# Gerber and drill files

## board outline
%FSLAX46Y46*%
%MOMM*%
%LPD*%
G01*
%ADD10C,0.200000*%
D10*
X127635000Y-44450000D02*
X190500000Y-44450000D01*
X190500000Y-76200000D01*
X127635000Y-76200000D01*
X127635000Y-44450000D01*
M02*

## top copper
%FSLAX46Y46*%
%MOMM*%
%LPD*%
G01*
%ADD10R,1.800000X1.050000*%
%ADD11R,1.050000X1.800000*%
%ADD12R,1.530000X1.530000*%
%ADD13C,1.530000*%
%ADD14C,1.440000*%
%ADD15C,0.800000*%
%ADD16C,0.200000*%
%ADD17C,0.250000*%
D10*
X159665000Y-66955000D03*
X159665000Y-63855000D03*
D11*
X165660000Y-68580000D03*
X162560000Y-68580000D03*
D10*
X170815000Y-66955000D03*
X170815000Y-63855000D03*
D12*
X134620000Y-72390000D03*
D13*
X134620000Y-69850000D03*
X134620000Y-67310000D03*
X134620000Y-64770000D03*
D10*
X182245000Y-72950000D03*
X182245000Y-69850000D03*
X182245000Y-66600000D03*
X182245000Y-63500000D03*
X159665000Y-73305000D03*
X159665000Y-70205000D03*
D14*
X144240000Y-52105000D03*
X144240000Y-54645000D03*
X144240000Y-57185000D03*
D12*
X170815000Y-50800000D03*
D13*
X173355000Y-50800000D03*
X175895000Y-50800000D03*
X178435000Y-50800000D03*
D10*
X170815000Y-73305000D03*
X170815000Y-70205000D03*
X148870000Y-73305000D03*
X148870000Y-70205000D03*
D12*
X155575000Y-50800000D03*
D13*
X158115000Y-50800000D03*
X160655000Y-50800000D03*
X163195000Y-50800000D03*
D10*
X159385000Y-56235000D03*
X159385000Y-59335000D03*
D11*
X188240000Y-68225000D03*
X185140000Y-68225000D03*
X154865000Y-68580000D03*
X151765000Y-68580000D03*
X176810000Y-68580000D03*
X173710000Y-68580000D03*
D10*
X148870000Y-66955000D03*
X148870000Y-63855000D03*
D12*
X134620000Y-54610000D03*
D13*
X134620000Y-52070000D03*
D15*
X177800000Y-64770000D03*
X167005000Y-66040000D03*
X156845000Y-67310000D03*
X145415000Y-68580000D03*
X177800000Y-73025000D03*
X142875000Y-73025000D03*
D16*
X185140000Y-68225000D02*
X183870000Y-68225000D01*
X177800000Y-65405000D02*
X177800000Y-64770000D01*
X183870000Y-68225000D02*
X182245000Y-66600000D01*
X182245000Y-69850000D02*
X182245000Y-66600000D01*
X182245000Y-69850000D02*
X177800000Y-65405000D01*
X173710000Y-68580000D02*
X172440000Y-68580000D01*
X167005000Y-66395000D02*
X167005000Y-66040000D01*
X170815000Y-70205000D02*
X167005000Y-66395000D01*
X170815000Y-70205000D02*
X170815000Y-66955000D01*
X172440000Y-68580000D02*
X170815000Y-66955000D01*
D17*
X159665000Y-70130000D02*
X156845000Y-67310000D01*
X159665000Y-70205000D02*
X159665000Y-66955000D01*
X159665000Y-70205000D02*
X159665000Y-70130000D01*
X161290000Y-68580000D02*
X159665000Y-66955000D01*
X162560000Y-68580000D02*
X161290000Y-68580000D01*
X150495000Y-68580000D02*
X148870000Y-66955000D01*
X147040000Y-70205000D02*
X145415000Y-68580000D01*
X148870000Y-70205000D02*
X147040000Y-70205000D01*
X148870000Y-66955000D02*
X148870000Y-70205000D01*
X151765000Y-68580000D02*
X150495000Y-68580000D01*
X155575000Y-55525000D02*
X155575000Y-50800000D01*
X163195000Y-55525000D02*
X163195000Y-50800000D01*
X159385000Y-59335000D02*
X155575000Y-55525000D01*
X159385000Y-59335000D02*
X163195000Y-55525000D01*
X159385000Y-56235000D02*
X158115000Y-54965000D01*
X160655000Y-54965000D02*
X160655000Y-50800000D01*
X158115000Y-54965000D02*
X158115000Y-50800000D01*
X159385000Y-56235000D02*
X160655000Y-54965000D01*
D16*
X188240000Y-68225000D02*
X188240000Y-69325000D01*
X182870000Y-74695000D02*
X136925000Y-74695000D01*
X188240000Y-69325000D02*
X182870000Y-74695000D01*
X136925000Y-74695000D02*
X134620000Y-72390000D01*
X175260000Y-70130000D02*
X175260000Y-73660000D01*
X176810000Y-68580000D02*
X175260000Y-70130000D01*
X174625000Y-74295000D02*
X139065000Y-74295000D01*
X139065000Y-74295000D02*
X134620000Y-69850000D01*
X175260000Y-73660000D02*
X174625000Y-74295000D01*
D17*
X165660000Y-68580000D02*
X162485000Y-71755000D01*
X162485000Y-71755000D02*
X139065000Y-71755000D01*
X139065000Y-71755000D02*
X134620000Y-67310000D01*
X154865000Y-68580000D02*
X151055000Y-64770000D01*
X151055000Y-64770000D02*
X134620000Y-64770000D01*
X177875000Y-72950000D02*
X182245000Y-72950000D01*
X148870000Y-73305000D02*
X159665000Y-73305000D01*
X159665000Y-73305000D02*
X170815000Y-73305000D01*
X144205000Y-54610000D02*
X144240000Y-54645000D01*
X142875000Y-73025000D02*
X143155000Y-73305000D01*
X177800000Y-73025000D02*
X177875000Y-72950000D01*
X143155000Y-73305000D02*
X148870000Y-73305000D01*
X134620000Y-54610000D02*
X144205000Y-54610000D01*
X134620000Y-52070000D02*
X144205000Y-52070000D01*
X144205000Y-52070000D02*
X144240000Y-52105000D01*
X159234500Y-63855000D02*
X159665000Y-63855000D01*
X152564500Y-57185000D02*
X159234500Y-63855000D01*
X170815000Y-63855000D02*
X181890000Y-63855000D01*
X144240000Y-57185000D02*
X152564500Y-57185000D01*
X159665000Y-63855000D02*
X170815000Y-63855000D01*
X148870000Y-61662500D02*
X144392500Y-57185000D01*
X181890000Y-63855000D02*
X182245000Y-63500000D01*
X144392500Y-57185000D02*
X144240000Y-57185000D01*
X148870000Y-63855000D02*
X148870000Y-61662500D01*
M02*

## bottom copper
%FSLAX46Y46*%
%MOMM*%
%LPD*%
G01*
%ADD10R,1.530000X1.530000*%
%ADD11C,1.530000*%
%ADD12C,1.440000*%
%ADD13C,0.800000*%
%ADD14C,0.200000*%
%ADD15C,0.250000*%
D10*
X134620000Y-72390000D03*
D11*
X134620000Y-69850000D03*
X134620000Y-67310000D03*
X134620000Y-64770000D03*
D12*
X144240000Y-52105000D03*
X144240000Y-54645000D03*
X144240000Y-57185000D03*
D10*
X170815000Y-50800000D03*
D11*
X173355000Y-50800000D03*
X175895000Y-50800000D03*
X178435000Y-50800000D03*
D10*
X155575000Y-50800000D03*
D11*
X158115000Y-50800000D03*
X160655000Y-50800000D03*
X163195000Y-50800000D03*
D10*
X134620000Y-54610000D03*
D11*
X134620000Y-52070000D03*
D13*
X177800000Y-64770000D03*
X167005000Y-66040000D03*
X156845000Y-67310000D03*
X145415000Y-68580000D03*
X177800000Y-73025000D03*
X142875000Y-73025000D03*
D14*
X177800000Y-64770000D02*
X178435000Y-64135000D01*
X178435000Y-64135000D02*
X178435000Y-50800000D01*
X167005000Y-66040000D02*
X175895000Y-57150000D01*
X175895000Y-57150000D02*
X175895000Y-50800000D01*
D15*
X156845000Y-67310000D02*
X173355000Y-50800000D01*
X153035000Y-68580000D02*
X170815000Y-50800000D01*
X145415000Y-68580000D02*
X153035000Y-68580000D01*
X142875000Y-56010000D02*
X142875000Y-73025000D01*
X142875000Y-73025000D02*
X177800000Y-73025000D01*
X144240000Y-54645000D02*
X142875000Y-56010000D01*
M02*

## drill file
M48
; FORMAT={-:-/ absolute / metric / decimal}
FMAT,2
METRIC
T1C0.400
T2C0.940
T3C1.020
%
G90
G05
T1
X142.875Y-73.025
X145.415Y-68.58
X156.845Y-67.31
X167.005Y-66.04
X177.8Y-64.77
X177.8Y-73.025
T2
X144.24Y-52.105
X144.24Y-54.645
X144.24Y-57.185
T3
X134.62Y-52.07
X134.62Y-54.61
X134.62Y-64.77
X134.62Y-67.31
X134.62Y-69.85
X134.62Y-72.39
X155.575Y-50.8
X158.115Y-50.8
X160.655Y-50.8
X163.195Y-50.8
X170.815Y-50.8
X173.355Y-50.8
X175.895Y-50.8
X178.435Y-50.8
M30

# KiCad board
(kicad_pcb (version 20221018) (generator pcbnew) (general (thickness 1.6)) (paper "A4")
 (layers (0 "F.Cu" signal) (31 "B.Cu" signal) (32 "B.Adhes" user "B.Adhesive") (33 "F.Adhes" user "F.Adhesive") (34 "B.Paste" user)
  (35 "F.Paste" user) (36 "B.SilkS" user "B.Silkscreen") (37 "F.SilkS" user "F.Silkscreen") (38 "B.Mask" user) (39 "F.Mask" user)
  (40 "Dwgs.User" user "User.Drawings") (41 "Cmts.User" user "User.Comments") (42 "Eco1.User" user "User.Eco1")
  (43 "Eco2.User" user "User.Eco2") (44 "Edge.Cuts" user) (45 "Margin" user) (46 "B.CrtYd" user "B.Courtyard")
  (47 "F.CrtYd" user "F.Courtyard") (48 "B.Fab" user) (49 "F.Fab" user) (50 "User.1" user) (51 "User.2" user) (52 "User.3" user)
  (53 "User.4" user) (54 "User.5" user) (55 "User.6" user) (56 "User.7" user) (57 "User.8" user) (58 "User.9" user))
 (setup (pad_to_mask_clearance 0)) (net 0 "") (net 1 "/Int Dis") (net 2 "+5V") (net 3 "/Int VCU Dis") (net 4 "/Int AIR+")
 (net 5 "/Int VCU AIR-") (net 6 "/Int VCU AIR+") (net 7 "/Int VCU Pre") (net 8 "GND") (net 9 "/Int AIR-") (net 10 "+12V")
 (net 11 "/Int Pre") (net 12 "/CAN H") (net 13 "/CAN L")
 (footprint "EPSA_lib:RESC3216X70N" (layer "F.Cu") (at 159.665 65.405 90)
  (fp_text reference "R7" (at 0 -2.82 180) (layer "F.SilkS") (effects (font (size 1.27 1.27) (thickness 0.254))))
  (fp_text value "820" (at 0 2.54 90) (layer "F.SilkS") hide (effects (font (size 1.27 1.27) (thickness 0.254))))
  (pad "1" smd rect (at -1.55 0 90) (size 1.05 1.8) (layers "F.Cu" "F.Paste" "F.Mask") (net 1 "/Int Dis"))
  (pad "2" smd rect (at 1.55 0 90) (size 1.05 1.8) (layers "F.Cu" "F.Paste" "F.Mask") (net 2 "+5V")))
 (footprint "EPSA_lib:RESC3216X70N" (layer "F.Cu") (at 164.11 68.58 180)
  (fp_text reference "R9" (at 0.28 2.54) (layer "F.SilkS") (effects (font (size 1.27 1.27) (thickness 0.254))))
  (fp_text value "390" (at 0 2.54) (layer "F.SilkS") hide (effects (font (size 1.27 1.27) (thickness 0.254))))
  (pad "1" smd rect (at -1.55 0 180) (size 1.05 1.8) (layers "F.Cu" "F.Paste" "F.Mask") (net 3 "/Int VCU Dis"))
  (pad "2" smd rect (at 1.55 0 180) (size 1.05 1.8) (layers "F.Cu" "F.Paste" "F.Mask") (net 1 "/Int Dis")))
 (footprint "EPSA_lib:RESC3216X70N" (layer "F.Cu") (at 170.815 65.405 90)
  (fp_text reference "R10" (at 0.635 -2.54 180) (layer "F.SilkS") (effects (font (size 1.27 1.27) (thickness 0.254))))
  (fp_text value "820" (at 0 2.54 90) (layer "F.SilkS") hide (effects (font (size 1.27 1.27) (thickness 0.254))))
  (pad "1" smd rect (at -1.55 0 90) (size 1.05 1.8) (layers "F.Cu" "F.Paste" "F.Mask") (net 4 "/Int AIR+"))
  (pad "2" smd rect (at 1.55 0 90) (size 1.05 1.8) (layers "F.Cu" "F.Paste" "F.Mask") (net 2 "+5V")))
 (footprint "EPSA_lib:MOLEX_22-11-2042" (layer "F.Cu") (at 134.62 68.58 90)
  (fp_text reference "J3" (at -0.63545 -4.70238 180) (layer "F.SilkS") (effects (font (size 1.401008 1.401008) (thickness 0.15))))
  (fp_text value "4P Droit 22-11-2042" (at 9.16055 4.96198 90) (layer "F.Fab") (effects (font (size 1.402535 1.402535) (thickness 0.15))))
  (pad "1" thru_hole rect (at -3.81 0 90) (size 1.53 1.53) (drill 1.02) (layers "*.Cu" "*.Mask") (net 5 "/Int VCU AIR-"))
  (pad "2" thru_hole circle (at -1.27 0 90) (size 1.53 1.53) (drill 1.02) (layers "*.Cu" "*.Mask") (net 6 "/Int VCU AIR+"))
  (pad "3" thru_hole circle (at 1.27 0 90) (size 1.53 1.53) (drill 1.02) (layers "*.Cu" "*.Mask") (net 3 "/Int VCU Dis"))
  (pad "4" thru_hole circle (at 3.81 0 90) (size 1.53 1.53) (drill 1.02) (layers "*.Cu" "*.Mask") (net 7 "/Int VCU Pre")))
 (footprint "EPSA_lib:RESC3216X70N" (layer "F.Cu") (at 182.245 71.4 90)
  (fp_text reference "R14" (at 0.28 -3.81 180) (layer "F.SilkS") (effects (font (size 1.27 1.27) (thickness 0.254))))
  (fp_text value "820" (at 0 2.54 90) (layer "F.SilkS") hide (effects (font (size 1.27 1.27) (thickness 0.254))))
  (pad "1" smd rect (at -1.55 0 90) (size 1.05 1.8) (layers "F.Cu" "F.Paste" "F.Mask") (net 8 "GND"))
  (pad "2" smd rect (at 1.55 0 90) (size 1.05 1.8) (layers "F.Cu" "F.Paste" "F.Mask") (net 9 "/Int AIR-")))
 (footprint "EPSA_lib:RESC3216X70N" (layer "F.Cu") (at 182.245 65.05 90)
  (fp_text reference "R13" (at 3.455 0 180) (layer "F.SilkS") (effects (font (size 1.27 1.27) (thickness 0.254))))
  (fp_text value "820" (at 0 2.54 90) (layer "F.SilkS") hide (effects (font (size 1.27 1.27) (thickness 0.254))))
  (pad "1" smd rect (at -1.55 0 90) (size 1.05 1.8) (layers "F.Cu" "F.Paste" "F.Mask") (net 9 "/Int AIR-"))
  (pad "2" smd rect (at 1.55 0 90) (size 1.05 1.8) (layers "F.Cu" "F.Paste" "F.Mask") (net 2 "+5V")))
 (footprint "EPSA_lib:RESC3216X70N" (layer "F.Cu") (at 159.665 71.755 90)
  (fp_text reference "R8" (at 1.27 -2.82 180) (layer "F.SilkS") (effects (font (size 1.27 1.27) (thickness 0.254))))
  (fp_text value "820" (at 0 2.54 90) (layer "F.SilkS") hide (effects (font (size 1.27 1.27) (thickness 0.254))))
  (pad "1" smd rect (at -1.55 0 90) (size 1.05 1.8) (layers "F.Cu" "F.Paste" "F.Mask") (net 8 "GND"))
  (pad "2" smd rect (at 1.55 0 90) (size 1.05 1.8) (layers "F.Cu" "F.Paste" "F.Mask") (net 1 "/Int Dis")))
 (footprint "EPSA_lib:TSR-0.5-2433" (layer "F.Cu") (at 142.24 48.895 -90)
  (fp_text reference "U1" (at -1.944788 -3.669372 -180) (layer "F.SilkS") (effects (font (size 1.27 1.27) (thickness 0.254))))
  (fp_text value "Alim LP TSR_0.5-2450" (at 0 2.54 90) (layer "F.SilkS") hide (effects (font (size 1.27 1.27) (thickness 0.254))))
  (pad "1" thru_hole circle (at 3.21 -2 270) (size 1.44 1.44) (drill 0.94) (layers "*.Cu" "*.Mask") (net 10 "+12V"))
  (pad "2" thru_hole circle (at 5.75 -2 270) (size 1.44 1.44) (drill 0.94) (layers "*.Cu" "*.Mask") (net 8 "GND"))
  (pad "3" thru_hole circle (at 8.29 -2 270) (size 1.44 1.44) (drill 0.94) (layers "*.Cu" "*.Mask") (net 2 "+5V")))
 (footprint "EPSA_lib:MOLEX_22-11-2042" (layer "F.Cu") (at 174.625 50.8)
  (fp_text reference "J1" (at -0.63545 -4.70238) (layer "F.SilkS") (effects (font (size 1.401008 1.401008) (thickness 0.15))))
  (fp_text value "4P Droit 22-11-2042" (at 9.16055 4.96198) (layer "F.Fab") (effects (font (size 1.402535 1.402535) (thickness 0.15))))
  (pad "1" thru_hole rect (at -3.81 0) (size 1.53 1.53) (drill 1.02) (layers "*.Cu" "*.Mask") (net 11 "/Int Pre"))
  (pad "2" thru_hole circle (at -1.27 0) (size 1.53 1.53) (drill 1.02) (layers "*.Cu" "*.Mask") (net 1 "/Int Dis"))
  (pad "3" thru_hole circle (at 1.27 0) (size 1.53 1.53) (drill 1.02) (layers "*.Cu" "*.Mask") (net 4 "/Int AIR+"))
  (pad "4" thru_hole circle (at 3.81 0) (size 1.53 1.53) (drill 1.02) (layers "*.Cu" "*.Mask") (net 9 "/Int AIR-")))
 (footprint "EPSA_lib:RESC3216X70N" (layer "F.Cu") (at 170.815 71.755 90)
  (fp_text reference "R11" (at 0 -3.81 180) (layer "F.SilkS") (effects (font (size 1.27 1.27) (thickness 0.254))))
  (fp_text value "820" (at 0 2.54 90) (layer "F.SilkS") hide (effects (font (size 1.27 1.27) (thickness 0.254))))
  (pad "1" smd rect (at -1.55 0 90) (size 1.05 1.8) (layers "F.Cu" "F.Paste" "F.Mask") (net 8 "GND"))
  (pad "2" smd rect (at 1.55 0 90) (size 1.05 1.8) (layers "F.Cu" "F.Paste" "F.Mask") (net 4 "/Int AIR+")))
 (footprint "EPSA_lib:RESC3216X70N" (layer "F.Cu") (at 148.87 71.755 90)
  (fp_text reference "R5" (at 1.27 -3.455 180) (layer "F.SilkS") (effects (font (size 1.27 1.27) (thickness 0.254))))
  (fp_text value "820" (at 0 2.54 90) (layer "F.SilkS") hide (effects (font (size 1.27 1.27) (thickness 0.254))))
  (pad "1" smd rect (at -1.55 0 90) (size 1.05 1.8) (layers "F.Cu" "F.Paste" "F.Mask") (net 8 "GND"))
  (pad "2" smd rect (at 1.55 0 90) (size 1.05 1.8) (layers "F.Cu" "F.Paste" "F.Mask") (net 11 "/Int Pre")))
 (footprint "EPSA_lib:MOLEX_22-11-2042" (layer "F.Cu") (at 159.385 50.8)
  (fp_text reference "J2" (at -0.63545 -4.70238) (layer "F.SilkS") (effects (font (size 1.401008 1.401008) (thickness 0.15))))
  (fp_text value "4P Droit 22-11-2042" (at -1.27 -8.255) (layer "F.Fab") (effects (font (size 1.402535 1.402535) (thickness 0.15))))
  (pad "1" thru_hole rect (at -3.81 0) (size 1.53 1.53) (drill 1.02) (layers "*.Cu" "*.Mask") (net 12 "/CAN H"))
  (pad "2" thru_hole circle (at -1.27 0) (size 1.53 1.53) (drill 1.02) (layers "*.Cu" "*.Mask") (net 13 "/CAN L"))
  (pad "3" thru_hole circle (at 1.27 0) (size 1.53 1.53) (drill 1.02) (layers "*.Cu" "*.Mask") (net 13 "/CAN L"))
  (pad "4" thru_hole circle (at 3.81 0) (size 1.53 1.53) (drill 1.02) (layers "*.Cu" "*.Mask") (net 12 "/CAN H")))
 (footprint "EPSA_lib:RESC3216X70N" (layer "F.Cu") (at 159.385 57.785 -90)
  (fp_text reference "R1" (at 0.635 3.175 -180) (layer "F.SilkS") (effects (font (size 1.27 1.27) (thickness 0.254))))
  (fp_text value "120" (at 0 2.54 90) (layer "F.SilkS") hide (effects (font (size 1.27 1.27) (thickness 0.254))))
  (pad "1" smd rect (at -1.55 0 270) (size 1.05 1.8) (layers "F.Cu" "F.Paste" "F.Mask") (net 13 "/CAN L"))
  (pad "2" smd rect (at 1.55 0 270) (size 1.05 1.8) (layers "F.Cu" "F.Paste" "F.Mask") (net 12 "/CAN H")))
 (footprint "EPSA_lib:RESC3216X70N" (layer "F.Cu") (at 186.69 68.225 180)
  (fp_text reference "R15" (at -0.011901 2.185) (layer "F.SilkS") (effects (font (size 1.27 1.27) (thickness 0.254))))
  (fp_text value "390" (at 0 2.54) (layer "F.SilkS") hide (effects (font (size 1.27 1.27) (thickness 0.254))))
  (pad "1" smd rect (at -1.55 0 180) (size 1.05 1.8) (layers "F.Cu" "F.Paste" "F.Mask") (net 5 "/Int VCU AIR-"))
  (pad "2" smd rect (at 1.55 0 180) (size 1.05 1.8) (layers "F.Cu" "F.Paste" "F.Mask") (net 9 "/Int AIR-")))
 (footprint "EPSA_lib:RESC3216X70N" (layer "F.Cu") (at 153.315 68.58 180)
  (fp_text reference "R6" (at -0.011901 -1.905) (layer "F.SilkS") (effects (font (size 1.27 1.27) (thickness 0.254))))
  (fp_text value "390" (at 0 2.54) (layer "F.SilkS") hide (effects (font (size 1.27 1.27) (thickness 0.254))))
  (pad "1" smd rect (at -1.55 0 180) (size 1.05 1.8) (layers "F.Cu" "F.Paste" "F.Mask") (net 7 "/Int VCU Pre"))
  (pad "2" smd rect (at 1.55 0 180) (size 1.05 1.8) (layers "F.Cu" "F.Paste" "F.Mask") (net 11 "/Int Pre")))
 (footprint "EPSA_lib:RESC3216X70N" (layer "F.Cu") (at 175.26 68.58 180)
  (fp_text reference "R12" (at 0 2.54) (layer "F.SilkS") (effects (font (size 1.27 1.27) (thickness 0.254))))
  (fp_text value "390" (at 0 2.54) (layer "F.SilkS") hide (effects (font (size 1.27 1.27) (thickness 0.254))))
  (pad "1" smd rect (at -1.55 0 180) (size 1.05 1.8) (layers "F.Cu" "F.Paste" "F.Mask") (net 6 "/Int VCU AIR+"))
  (pad "2" smd rect (at 1.55 0 180) (size 1.05 1.8) (layers "F.Cu" "F.Paste" "F.Mask") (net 4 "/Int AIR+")))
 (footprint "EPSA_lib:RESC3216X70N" (layer "F.Cu") (at 148.87 65.405 90)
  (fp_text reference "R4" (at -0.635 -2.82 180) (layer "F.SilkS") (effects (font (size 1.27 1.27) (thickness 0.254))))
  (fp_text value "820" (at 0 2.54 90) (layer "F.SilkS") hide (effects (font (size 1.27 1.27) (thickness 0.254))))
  (pad "1" smd rect (at -1.55 0 90) (size 1.05 1.8) (layers "F.Cu" "F.Paste" "F.Mask") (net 11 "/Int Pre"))
  (pad "2" smd rect (at 1.55 0 90) (size 1.05 1.8) (layers "F.Cu" "F.Paste" "F.Mask") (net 2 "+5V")))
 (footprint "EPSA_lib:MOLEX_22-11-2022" (layer "F.Cu") (at 134.62 54.61 90)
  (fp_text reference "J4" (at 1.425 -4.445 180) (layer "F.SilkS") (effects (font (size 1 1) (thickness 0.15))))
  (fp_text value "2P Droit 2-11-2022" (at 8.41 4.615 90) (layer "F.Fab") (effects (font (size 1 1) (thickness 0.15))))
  (pad "1" thru_hole rect (at 0 0 90) (size 1.53 1.53) (drill 1.02) (layers "*.Cu" "*.Mask") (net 8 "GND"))
  (pad "2" thru_hole circle (at 2.54 0 90) (size 1.53 1.53) (drill 1.02) (layers "*.Cu" "*.Mask") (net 10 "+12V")))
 (gr_rect (start 127.635 44.45) (end 190.5 76.2) (stroke (width 0.2) (type default)) (fill none) (layer "Edge.Cuts"))
 (segment (start 185.14 68.225) (end 183.87 68.225) (width 0.2) (layer "F.Cu") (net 9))
 (segment (start 177.8 65.405) (end 177.8 64.77) (width 0.2) (layer "F.Cu") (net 9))
 (segment (start 183.87 68.225) (end 182.245 66.6) (width 0.2) (layer "F.Cu") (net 9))
 (segment (start 182.245 69.85) (end 182.245 66.6) (width 0.2) (layer "F.Cu") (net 9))
 (segment (start 182.245 69.85) (end 177.8 65.405) (width 0.2) (layer "F.Cu") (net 9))
 (via (at 177.8 64.77) (size 0.8) (drill 0.4) (layers "F.Cu" "B.Cu") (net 9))
 (segment (start 177.8 64.77) (end 178.435 64.135) (width 0.2) (layer "B.Cu") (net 9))
 (segment (start 178.435 64.135) (end 178.435 50.8) (width 0.2) (layer "B.Cu") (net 9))
 (segment (start 173.71 68.58) (end 172.44 68.58) (width 0.2) (layer "F.Cu") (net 4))
 (segment (start 167.005 66.395) (end 167.005 66.04) (width 0.2) (layer "F.Cu") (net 4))
 (segment (start 170.815 70.205) (end 167.005 66.395) (width 0.2) (layer "F.Cu") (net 4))
 (segment (start 170.815 70.205) (end 170.815 66.955) (width 0.2) (layer "F.Cu") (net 4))
 (segment (start 172.44 68.58) (end 170.815 66.955) (width 0.2) (layer "F.Cu") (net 4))
 (via (at 167.005 66.04) (size 0.8) (drill 0.4) (layers "F.Cu" "B.Cu") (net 4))
 (segment (start 167.005 66.04) (end 175.895 57.15) (width 0.2) (layer "B.Cu") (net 4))
 (segment (start 175.895 57.15) (end 175.895 50.8) (width 0.2) (layer "B.Cu") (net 4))
 (segment (start 159.665 70.13) (end 156.845 67.31) (width 0.25) (layer "F.Cu") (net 1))
 (segment (start 159.665 70.205) (end 159.665 66.955) (width 0.25) (layer "F.Cu") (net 1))
 (segment (start 159.665 70.205) (end 159.665 70.13) (width 0.25) (layer "F.Cu") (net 1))
 (segment (start 161.29 68.58) (end 159.665 66.955) (width 0.25) (layer "F.Cu") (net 1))
 (segment (start 162.56 68.58) (end 161.29 68.58) (width 0.25) (layer "F.Cu") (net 1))
 (via (at 156.845 67.31) (size 0.8) (drill 0.4) (layers "F.Cu" "B.Cu") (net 1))
 (segment (start 156.845 67.31) (end 173.355 50.8) (width 0.25) (layer "B.Cu") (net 1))
 (segment (start 150.495 68.58) (end 148.87 66.955) (width 0.25) (layer "F.Cu") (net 11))
 (segment (start 147.04 70.205) (end 145.415 68.58) (width 0.25) (layer "F.Cu") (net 11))
 (segment (start 148.87 70.205) (end 147.04 70.205) (width 0.25) (layer "F.Cu") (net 11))
 (segment (start 148.87 66.955) (end 148.87 70.205) (width 0.25) (layer "F.Cu") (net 11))
 (segment (start 151.765 68.58) (end 150.495 68.58) (width 0.25) (layer "F.Cu") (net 11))
 (via (at 145.415 68.58) (size 0.8) (drill 0.4) (layers "F.Cu" "B.Cu") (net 11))
 (segment (start 153.035 68.58) (end 170.815 50.8) (width 0.25) (layer "B.Cu") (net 11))
 (segment (start 145.415 68.58) (end 153.035 68.58) (width 0.25) (layer "B.Cu") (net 11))
 (segment (start 155.575 55.525) (end 155.575 50.8) (width 0.25) (layer "F.Cu") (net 12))
 (segment (start 163.195 55.525) (end 163.195 50.8) (width 0.25) (layer "F.Cu") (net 12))
 (segment (start 159.385 59.335) (end 155.575 55.525) (width 0.25) (layer "F.Cu") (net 12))
 (segment (start 159.385 59.335) (end 163.195 55.525) (width 0.25) (layer "F.Cu") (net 12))
 (segment (start 159.385 56.235) (end 158.115 54.965) (width 0.25) (layer "F.Cu") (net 13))
 (segment (start 160.655 54.965) (end 160.655 50.8) (width 0.25) (layer "F.Cu") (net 13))
 (segment (start 158.115 54.965) (end 158.115 50.8) (width 0.25) (layer "F.Cu") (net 13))
 (segment (start 159.385 56.235) (end 160.655 54.965) (width 0.25) (layer "F.Cu") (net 13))
 (segment (start 188.24 68.225) (end 188.24 69.325) (width 0.2) (layer "F.Cu") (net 5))
 (segment (start 182.87 74.695) (end 136.925 74.695) (width 0.2) (layer "F.Cu") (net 5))
 (segment (start 188.24 69.325) (end 182.87 74.695) (width 0.2) (layer "F.Cu") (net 5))
 (segment (start 136.925 74.695) (end 134.62 72.39) (width 0.2) (layer "F.Cu") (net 5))
 (segment (start 175.26 70.13) (end 175.26 73.66) (width 0.2) (layer "F.Cu") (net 6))
 (segment (start 176.81 68.58) (end 175.26 70.13) (width 0.2) (layer "F.Cu") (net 6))
 (segment (start 174.625 74.295) (end 139.065 74.295) (width 0.2) (layer "F.Cu") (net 6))
 (segment (start 139.065 74.295) (end 134.62 69.85) (width 0.2) (layer "F.Cu") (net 6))
 (segment (start 175.26 73.66) (end 174.625 74.295) (width 0.2) (layer "F.Cu") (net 6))
 (segment (start 165.66 68.58) (end 162.485 71.755) (width 0.25) (layer "F.Cu") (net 3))
 (segment (start 162.485 71.755) (end 139.065 71.755) (width 0.25) (layer "F.Cu") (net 3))
 (segment (start 139.065 71.755) (end 134.62 67.31) (width 0.25) (layer "F.Cu") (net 3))
 (segment (start 154.865 68.58) (end 151.055 64.77) (width 0.25) (layer "F.Cu") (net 7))
 (segment (start 151.055 64.77) (end 134.62 64.77) (width 0.25) (layer "F.Cu") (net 7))
 (segment (start 177.875 72.95) (end 182.245 72.95) (width 0.25) (layer "F.Cu") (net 8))
 (segment (start 148.87 73.305) (end 159.665 73.305) (width 0.25) (layer "F.Cu") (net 8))
 (segment (start 159.665 73.305) (end 170.815 73.305) (width 0.25) (layer "F.Cu") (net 8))
 (segment (start 144.205 54.61) (end 144.24 54.645) (width 0.25) (layer "F.Cu") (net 8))
 (segment (start 142.875 73.025) (end 143.155 73.305) (width 0.25) (layer "F.Cu") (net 8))
 (segment (start 177.8 73.025) (end 177.875 72.95) (width 0.25) (layer "F.Cu") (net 8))
 (segment (start 143.155 73.305) (end 148.87 73.305) (width 0.25) (layer "F.Cu") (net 8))
 (segment (start 134.62 54.61) (end 144.205 54.61) (width 0.25) (layer "F.Cu") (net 8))
 (via (at 177.8 73.025) (size 0.8) (drill 0.4) (layers "F.Cu" "B.Cu") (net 8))
 (via (at 142.875 73.025) (size 0.8) (drill 0.4) (layers "F.Cu" "B.Cu") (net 8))
 (segment (start 142.875 56.01) (end 142.875 73.025) (width 0.25) (layer "B.Cu") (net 8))
 (segment (start 142.875 73.025) (end 177.8 73.025) (width 0.25) (layer "B.Cu") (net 8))
 (segment (start 144.24 54.645) (end 142.875 56.01) (width 0.25) (layer "B.Cu") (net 8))
 (segment (start 134.62 52.07) (end 144.205 52.07) (width 0.25) (layer "F.Cu") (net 10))
 (segment (start 144.205 52.07) (end 144.24 52.105) (width 0.25) (layer "F.Cu") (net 10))
 (segment (start 159.2345 63.855) (end 159.665 63.855) (width 0.25) (layer "F.Cu") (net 2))
 (segment (start 152.5645 57.185) (end 159.2345 63.855) (width 0.25) (layer "F.Cu") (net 2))
 (segment (start 170.815 63.855) (end 181.89 63.855) (width 0.25) (layer "F.Cu") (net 2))
 (segment (start 144.24 57.185) (end 152.5645 57.185) (width 0.25) (layer "F.Cu") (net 2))
 (segment (start 159.665 63.855) (end 170.815 63.855) (width 0.25) (layer "F.Cu") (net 2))
 (segment (start 148.87 61.6625) (end 144.3925 57.185) (width 0.25) (layer "F.Cu") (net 2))
 (segment (start 181.89 63.855) (end 182.245 63.5) (width 0.25) (layer "F.Cu") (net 2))
 (segment (start 144.3925 57.185) (end 144.24 57.185) (width 0.25) (layer "F.Cu") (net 2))
 (segment (start 148.87 63.855) (end 148.87 61.6625) (width 0.25) (layer "F.Cu") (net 2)))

